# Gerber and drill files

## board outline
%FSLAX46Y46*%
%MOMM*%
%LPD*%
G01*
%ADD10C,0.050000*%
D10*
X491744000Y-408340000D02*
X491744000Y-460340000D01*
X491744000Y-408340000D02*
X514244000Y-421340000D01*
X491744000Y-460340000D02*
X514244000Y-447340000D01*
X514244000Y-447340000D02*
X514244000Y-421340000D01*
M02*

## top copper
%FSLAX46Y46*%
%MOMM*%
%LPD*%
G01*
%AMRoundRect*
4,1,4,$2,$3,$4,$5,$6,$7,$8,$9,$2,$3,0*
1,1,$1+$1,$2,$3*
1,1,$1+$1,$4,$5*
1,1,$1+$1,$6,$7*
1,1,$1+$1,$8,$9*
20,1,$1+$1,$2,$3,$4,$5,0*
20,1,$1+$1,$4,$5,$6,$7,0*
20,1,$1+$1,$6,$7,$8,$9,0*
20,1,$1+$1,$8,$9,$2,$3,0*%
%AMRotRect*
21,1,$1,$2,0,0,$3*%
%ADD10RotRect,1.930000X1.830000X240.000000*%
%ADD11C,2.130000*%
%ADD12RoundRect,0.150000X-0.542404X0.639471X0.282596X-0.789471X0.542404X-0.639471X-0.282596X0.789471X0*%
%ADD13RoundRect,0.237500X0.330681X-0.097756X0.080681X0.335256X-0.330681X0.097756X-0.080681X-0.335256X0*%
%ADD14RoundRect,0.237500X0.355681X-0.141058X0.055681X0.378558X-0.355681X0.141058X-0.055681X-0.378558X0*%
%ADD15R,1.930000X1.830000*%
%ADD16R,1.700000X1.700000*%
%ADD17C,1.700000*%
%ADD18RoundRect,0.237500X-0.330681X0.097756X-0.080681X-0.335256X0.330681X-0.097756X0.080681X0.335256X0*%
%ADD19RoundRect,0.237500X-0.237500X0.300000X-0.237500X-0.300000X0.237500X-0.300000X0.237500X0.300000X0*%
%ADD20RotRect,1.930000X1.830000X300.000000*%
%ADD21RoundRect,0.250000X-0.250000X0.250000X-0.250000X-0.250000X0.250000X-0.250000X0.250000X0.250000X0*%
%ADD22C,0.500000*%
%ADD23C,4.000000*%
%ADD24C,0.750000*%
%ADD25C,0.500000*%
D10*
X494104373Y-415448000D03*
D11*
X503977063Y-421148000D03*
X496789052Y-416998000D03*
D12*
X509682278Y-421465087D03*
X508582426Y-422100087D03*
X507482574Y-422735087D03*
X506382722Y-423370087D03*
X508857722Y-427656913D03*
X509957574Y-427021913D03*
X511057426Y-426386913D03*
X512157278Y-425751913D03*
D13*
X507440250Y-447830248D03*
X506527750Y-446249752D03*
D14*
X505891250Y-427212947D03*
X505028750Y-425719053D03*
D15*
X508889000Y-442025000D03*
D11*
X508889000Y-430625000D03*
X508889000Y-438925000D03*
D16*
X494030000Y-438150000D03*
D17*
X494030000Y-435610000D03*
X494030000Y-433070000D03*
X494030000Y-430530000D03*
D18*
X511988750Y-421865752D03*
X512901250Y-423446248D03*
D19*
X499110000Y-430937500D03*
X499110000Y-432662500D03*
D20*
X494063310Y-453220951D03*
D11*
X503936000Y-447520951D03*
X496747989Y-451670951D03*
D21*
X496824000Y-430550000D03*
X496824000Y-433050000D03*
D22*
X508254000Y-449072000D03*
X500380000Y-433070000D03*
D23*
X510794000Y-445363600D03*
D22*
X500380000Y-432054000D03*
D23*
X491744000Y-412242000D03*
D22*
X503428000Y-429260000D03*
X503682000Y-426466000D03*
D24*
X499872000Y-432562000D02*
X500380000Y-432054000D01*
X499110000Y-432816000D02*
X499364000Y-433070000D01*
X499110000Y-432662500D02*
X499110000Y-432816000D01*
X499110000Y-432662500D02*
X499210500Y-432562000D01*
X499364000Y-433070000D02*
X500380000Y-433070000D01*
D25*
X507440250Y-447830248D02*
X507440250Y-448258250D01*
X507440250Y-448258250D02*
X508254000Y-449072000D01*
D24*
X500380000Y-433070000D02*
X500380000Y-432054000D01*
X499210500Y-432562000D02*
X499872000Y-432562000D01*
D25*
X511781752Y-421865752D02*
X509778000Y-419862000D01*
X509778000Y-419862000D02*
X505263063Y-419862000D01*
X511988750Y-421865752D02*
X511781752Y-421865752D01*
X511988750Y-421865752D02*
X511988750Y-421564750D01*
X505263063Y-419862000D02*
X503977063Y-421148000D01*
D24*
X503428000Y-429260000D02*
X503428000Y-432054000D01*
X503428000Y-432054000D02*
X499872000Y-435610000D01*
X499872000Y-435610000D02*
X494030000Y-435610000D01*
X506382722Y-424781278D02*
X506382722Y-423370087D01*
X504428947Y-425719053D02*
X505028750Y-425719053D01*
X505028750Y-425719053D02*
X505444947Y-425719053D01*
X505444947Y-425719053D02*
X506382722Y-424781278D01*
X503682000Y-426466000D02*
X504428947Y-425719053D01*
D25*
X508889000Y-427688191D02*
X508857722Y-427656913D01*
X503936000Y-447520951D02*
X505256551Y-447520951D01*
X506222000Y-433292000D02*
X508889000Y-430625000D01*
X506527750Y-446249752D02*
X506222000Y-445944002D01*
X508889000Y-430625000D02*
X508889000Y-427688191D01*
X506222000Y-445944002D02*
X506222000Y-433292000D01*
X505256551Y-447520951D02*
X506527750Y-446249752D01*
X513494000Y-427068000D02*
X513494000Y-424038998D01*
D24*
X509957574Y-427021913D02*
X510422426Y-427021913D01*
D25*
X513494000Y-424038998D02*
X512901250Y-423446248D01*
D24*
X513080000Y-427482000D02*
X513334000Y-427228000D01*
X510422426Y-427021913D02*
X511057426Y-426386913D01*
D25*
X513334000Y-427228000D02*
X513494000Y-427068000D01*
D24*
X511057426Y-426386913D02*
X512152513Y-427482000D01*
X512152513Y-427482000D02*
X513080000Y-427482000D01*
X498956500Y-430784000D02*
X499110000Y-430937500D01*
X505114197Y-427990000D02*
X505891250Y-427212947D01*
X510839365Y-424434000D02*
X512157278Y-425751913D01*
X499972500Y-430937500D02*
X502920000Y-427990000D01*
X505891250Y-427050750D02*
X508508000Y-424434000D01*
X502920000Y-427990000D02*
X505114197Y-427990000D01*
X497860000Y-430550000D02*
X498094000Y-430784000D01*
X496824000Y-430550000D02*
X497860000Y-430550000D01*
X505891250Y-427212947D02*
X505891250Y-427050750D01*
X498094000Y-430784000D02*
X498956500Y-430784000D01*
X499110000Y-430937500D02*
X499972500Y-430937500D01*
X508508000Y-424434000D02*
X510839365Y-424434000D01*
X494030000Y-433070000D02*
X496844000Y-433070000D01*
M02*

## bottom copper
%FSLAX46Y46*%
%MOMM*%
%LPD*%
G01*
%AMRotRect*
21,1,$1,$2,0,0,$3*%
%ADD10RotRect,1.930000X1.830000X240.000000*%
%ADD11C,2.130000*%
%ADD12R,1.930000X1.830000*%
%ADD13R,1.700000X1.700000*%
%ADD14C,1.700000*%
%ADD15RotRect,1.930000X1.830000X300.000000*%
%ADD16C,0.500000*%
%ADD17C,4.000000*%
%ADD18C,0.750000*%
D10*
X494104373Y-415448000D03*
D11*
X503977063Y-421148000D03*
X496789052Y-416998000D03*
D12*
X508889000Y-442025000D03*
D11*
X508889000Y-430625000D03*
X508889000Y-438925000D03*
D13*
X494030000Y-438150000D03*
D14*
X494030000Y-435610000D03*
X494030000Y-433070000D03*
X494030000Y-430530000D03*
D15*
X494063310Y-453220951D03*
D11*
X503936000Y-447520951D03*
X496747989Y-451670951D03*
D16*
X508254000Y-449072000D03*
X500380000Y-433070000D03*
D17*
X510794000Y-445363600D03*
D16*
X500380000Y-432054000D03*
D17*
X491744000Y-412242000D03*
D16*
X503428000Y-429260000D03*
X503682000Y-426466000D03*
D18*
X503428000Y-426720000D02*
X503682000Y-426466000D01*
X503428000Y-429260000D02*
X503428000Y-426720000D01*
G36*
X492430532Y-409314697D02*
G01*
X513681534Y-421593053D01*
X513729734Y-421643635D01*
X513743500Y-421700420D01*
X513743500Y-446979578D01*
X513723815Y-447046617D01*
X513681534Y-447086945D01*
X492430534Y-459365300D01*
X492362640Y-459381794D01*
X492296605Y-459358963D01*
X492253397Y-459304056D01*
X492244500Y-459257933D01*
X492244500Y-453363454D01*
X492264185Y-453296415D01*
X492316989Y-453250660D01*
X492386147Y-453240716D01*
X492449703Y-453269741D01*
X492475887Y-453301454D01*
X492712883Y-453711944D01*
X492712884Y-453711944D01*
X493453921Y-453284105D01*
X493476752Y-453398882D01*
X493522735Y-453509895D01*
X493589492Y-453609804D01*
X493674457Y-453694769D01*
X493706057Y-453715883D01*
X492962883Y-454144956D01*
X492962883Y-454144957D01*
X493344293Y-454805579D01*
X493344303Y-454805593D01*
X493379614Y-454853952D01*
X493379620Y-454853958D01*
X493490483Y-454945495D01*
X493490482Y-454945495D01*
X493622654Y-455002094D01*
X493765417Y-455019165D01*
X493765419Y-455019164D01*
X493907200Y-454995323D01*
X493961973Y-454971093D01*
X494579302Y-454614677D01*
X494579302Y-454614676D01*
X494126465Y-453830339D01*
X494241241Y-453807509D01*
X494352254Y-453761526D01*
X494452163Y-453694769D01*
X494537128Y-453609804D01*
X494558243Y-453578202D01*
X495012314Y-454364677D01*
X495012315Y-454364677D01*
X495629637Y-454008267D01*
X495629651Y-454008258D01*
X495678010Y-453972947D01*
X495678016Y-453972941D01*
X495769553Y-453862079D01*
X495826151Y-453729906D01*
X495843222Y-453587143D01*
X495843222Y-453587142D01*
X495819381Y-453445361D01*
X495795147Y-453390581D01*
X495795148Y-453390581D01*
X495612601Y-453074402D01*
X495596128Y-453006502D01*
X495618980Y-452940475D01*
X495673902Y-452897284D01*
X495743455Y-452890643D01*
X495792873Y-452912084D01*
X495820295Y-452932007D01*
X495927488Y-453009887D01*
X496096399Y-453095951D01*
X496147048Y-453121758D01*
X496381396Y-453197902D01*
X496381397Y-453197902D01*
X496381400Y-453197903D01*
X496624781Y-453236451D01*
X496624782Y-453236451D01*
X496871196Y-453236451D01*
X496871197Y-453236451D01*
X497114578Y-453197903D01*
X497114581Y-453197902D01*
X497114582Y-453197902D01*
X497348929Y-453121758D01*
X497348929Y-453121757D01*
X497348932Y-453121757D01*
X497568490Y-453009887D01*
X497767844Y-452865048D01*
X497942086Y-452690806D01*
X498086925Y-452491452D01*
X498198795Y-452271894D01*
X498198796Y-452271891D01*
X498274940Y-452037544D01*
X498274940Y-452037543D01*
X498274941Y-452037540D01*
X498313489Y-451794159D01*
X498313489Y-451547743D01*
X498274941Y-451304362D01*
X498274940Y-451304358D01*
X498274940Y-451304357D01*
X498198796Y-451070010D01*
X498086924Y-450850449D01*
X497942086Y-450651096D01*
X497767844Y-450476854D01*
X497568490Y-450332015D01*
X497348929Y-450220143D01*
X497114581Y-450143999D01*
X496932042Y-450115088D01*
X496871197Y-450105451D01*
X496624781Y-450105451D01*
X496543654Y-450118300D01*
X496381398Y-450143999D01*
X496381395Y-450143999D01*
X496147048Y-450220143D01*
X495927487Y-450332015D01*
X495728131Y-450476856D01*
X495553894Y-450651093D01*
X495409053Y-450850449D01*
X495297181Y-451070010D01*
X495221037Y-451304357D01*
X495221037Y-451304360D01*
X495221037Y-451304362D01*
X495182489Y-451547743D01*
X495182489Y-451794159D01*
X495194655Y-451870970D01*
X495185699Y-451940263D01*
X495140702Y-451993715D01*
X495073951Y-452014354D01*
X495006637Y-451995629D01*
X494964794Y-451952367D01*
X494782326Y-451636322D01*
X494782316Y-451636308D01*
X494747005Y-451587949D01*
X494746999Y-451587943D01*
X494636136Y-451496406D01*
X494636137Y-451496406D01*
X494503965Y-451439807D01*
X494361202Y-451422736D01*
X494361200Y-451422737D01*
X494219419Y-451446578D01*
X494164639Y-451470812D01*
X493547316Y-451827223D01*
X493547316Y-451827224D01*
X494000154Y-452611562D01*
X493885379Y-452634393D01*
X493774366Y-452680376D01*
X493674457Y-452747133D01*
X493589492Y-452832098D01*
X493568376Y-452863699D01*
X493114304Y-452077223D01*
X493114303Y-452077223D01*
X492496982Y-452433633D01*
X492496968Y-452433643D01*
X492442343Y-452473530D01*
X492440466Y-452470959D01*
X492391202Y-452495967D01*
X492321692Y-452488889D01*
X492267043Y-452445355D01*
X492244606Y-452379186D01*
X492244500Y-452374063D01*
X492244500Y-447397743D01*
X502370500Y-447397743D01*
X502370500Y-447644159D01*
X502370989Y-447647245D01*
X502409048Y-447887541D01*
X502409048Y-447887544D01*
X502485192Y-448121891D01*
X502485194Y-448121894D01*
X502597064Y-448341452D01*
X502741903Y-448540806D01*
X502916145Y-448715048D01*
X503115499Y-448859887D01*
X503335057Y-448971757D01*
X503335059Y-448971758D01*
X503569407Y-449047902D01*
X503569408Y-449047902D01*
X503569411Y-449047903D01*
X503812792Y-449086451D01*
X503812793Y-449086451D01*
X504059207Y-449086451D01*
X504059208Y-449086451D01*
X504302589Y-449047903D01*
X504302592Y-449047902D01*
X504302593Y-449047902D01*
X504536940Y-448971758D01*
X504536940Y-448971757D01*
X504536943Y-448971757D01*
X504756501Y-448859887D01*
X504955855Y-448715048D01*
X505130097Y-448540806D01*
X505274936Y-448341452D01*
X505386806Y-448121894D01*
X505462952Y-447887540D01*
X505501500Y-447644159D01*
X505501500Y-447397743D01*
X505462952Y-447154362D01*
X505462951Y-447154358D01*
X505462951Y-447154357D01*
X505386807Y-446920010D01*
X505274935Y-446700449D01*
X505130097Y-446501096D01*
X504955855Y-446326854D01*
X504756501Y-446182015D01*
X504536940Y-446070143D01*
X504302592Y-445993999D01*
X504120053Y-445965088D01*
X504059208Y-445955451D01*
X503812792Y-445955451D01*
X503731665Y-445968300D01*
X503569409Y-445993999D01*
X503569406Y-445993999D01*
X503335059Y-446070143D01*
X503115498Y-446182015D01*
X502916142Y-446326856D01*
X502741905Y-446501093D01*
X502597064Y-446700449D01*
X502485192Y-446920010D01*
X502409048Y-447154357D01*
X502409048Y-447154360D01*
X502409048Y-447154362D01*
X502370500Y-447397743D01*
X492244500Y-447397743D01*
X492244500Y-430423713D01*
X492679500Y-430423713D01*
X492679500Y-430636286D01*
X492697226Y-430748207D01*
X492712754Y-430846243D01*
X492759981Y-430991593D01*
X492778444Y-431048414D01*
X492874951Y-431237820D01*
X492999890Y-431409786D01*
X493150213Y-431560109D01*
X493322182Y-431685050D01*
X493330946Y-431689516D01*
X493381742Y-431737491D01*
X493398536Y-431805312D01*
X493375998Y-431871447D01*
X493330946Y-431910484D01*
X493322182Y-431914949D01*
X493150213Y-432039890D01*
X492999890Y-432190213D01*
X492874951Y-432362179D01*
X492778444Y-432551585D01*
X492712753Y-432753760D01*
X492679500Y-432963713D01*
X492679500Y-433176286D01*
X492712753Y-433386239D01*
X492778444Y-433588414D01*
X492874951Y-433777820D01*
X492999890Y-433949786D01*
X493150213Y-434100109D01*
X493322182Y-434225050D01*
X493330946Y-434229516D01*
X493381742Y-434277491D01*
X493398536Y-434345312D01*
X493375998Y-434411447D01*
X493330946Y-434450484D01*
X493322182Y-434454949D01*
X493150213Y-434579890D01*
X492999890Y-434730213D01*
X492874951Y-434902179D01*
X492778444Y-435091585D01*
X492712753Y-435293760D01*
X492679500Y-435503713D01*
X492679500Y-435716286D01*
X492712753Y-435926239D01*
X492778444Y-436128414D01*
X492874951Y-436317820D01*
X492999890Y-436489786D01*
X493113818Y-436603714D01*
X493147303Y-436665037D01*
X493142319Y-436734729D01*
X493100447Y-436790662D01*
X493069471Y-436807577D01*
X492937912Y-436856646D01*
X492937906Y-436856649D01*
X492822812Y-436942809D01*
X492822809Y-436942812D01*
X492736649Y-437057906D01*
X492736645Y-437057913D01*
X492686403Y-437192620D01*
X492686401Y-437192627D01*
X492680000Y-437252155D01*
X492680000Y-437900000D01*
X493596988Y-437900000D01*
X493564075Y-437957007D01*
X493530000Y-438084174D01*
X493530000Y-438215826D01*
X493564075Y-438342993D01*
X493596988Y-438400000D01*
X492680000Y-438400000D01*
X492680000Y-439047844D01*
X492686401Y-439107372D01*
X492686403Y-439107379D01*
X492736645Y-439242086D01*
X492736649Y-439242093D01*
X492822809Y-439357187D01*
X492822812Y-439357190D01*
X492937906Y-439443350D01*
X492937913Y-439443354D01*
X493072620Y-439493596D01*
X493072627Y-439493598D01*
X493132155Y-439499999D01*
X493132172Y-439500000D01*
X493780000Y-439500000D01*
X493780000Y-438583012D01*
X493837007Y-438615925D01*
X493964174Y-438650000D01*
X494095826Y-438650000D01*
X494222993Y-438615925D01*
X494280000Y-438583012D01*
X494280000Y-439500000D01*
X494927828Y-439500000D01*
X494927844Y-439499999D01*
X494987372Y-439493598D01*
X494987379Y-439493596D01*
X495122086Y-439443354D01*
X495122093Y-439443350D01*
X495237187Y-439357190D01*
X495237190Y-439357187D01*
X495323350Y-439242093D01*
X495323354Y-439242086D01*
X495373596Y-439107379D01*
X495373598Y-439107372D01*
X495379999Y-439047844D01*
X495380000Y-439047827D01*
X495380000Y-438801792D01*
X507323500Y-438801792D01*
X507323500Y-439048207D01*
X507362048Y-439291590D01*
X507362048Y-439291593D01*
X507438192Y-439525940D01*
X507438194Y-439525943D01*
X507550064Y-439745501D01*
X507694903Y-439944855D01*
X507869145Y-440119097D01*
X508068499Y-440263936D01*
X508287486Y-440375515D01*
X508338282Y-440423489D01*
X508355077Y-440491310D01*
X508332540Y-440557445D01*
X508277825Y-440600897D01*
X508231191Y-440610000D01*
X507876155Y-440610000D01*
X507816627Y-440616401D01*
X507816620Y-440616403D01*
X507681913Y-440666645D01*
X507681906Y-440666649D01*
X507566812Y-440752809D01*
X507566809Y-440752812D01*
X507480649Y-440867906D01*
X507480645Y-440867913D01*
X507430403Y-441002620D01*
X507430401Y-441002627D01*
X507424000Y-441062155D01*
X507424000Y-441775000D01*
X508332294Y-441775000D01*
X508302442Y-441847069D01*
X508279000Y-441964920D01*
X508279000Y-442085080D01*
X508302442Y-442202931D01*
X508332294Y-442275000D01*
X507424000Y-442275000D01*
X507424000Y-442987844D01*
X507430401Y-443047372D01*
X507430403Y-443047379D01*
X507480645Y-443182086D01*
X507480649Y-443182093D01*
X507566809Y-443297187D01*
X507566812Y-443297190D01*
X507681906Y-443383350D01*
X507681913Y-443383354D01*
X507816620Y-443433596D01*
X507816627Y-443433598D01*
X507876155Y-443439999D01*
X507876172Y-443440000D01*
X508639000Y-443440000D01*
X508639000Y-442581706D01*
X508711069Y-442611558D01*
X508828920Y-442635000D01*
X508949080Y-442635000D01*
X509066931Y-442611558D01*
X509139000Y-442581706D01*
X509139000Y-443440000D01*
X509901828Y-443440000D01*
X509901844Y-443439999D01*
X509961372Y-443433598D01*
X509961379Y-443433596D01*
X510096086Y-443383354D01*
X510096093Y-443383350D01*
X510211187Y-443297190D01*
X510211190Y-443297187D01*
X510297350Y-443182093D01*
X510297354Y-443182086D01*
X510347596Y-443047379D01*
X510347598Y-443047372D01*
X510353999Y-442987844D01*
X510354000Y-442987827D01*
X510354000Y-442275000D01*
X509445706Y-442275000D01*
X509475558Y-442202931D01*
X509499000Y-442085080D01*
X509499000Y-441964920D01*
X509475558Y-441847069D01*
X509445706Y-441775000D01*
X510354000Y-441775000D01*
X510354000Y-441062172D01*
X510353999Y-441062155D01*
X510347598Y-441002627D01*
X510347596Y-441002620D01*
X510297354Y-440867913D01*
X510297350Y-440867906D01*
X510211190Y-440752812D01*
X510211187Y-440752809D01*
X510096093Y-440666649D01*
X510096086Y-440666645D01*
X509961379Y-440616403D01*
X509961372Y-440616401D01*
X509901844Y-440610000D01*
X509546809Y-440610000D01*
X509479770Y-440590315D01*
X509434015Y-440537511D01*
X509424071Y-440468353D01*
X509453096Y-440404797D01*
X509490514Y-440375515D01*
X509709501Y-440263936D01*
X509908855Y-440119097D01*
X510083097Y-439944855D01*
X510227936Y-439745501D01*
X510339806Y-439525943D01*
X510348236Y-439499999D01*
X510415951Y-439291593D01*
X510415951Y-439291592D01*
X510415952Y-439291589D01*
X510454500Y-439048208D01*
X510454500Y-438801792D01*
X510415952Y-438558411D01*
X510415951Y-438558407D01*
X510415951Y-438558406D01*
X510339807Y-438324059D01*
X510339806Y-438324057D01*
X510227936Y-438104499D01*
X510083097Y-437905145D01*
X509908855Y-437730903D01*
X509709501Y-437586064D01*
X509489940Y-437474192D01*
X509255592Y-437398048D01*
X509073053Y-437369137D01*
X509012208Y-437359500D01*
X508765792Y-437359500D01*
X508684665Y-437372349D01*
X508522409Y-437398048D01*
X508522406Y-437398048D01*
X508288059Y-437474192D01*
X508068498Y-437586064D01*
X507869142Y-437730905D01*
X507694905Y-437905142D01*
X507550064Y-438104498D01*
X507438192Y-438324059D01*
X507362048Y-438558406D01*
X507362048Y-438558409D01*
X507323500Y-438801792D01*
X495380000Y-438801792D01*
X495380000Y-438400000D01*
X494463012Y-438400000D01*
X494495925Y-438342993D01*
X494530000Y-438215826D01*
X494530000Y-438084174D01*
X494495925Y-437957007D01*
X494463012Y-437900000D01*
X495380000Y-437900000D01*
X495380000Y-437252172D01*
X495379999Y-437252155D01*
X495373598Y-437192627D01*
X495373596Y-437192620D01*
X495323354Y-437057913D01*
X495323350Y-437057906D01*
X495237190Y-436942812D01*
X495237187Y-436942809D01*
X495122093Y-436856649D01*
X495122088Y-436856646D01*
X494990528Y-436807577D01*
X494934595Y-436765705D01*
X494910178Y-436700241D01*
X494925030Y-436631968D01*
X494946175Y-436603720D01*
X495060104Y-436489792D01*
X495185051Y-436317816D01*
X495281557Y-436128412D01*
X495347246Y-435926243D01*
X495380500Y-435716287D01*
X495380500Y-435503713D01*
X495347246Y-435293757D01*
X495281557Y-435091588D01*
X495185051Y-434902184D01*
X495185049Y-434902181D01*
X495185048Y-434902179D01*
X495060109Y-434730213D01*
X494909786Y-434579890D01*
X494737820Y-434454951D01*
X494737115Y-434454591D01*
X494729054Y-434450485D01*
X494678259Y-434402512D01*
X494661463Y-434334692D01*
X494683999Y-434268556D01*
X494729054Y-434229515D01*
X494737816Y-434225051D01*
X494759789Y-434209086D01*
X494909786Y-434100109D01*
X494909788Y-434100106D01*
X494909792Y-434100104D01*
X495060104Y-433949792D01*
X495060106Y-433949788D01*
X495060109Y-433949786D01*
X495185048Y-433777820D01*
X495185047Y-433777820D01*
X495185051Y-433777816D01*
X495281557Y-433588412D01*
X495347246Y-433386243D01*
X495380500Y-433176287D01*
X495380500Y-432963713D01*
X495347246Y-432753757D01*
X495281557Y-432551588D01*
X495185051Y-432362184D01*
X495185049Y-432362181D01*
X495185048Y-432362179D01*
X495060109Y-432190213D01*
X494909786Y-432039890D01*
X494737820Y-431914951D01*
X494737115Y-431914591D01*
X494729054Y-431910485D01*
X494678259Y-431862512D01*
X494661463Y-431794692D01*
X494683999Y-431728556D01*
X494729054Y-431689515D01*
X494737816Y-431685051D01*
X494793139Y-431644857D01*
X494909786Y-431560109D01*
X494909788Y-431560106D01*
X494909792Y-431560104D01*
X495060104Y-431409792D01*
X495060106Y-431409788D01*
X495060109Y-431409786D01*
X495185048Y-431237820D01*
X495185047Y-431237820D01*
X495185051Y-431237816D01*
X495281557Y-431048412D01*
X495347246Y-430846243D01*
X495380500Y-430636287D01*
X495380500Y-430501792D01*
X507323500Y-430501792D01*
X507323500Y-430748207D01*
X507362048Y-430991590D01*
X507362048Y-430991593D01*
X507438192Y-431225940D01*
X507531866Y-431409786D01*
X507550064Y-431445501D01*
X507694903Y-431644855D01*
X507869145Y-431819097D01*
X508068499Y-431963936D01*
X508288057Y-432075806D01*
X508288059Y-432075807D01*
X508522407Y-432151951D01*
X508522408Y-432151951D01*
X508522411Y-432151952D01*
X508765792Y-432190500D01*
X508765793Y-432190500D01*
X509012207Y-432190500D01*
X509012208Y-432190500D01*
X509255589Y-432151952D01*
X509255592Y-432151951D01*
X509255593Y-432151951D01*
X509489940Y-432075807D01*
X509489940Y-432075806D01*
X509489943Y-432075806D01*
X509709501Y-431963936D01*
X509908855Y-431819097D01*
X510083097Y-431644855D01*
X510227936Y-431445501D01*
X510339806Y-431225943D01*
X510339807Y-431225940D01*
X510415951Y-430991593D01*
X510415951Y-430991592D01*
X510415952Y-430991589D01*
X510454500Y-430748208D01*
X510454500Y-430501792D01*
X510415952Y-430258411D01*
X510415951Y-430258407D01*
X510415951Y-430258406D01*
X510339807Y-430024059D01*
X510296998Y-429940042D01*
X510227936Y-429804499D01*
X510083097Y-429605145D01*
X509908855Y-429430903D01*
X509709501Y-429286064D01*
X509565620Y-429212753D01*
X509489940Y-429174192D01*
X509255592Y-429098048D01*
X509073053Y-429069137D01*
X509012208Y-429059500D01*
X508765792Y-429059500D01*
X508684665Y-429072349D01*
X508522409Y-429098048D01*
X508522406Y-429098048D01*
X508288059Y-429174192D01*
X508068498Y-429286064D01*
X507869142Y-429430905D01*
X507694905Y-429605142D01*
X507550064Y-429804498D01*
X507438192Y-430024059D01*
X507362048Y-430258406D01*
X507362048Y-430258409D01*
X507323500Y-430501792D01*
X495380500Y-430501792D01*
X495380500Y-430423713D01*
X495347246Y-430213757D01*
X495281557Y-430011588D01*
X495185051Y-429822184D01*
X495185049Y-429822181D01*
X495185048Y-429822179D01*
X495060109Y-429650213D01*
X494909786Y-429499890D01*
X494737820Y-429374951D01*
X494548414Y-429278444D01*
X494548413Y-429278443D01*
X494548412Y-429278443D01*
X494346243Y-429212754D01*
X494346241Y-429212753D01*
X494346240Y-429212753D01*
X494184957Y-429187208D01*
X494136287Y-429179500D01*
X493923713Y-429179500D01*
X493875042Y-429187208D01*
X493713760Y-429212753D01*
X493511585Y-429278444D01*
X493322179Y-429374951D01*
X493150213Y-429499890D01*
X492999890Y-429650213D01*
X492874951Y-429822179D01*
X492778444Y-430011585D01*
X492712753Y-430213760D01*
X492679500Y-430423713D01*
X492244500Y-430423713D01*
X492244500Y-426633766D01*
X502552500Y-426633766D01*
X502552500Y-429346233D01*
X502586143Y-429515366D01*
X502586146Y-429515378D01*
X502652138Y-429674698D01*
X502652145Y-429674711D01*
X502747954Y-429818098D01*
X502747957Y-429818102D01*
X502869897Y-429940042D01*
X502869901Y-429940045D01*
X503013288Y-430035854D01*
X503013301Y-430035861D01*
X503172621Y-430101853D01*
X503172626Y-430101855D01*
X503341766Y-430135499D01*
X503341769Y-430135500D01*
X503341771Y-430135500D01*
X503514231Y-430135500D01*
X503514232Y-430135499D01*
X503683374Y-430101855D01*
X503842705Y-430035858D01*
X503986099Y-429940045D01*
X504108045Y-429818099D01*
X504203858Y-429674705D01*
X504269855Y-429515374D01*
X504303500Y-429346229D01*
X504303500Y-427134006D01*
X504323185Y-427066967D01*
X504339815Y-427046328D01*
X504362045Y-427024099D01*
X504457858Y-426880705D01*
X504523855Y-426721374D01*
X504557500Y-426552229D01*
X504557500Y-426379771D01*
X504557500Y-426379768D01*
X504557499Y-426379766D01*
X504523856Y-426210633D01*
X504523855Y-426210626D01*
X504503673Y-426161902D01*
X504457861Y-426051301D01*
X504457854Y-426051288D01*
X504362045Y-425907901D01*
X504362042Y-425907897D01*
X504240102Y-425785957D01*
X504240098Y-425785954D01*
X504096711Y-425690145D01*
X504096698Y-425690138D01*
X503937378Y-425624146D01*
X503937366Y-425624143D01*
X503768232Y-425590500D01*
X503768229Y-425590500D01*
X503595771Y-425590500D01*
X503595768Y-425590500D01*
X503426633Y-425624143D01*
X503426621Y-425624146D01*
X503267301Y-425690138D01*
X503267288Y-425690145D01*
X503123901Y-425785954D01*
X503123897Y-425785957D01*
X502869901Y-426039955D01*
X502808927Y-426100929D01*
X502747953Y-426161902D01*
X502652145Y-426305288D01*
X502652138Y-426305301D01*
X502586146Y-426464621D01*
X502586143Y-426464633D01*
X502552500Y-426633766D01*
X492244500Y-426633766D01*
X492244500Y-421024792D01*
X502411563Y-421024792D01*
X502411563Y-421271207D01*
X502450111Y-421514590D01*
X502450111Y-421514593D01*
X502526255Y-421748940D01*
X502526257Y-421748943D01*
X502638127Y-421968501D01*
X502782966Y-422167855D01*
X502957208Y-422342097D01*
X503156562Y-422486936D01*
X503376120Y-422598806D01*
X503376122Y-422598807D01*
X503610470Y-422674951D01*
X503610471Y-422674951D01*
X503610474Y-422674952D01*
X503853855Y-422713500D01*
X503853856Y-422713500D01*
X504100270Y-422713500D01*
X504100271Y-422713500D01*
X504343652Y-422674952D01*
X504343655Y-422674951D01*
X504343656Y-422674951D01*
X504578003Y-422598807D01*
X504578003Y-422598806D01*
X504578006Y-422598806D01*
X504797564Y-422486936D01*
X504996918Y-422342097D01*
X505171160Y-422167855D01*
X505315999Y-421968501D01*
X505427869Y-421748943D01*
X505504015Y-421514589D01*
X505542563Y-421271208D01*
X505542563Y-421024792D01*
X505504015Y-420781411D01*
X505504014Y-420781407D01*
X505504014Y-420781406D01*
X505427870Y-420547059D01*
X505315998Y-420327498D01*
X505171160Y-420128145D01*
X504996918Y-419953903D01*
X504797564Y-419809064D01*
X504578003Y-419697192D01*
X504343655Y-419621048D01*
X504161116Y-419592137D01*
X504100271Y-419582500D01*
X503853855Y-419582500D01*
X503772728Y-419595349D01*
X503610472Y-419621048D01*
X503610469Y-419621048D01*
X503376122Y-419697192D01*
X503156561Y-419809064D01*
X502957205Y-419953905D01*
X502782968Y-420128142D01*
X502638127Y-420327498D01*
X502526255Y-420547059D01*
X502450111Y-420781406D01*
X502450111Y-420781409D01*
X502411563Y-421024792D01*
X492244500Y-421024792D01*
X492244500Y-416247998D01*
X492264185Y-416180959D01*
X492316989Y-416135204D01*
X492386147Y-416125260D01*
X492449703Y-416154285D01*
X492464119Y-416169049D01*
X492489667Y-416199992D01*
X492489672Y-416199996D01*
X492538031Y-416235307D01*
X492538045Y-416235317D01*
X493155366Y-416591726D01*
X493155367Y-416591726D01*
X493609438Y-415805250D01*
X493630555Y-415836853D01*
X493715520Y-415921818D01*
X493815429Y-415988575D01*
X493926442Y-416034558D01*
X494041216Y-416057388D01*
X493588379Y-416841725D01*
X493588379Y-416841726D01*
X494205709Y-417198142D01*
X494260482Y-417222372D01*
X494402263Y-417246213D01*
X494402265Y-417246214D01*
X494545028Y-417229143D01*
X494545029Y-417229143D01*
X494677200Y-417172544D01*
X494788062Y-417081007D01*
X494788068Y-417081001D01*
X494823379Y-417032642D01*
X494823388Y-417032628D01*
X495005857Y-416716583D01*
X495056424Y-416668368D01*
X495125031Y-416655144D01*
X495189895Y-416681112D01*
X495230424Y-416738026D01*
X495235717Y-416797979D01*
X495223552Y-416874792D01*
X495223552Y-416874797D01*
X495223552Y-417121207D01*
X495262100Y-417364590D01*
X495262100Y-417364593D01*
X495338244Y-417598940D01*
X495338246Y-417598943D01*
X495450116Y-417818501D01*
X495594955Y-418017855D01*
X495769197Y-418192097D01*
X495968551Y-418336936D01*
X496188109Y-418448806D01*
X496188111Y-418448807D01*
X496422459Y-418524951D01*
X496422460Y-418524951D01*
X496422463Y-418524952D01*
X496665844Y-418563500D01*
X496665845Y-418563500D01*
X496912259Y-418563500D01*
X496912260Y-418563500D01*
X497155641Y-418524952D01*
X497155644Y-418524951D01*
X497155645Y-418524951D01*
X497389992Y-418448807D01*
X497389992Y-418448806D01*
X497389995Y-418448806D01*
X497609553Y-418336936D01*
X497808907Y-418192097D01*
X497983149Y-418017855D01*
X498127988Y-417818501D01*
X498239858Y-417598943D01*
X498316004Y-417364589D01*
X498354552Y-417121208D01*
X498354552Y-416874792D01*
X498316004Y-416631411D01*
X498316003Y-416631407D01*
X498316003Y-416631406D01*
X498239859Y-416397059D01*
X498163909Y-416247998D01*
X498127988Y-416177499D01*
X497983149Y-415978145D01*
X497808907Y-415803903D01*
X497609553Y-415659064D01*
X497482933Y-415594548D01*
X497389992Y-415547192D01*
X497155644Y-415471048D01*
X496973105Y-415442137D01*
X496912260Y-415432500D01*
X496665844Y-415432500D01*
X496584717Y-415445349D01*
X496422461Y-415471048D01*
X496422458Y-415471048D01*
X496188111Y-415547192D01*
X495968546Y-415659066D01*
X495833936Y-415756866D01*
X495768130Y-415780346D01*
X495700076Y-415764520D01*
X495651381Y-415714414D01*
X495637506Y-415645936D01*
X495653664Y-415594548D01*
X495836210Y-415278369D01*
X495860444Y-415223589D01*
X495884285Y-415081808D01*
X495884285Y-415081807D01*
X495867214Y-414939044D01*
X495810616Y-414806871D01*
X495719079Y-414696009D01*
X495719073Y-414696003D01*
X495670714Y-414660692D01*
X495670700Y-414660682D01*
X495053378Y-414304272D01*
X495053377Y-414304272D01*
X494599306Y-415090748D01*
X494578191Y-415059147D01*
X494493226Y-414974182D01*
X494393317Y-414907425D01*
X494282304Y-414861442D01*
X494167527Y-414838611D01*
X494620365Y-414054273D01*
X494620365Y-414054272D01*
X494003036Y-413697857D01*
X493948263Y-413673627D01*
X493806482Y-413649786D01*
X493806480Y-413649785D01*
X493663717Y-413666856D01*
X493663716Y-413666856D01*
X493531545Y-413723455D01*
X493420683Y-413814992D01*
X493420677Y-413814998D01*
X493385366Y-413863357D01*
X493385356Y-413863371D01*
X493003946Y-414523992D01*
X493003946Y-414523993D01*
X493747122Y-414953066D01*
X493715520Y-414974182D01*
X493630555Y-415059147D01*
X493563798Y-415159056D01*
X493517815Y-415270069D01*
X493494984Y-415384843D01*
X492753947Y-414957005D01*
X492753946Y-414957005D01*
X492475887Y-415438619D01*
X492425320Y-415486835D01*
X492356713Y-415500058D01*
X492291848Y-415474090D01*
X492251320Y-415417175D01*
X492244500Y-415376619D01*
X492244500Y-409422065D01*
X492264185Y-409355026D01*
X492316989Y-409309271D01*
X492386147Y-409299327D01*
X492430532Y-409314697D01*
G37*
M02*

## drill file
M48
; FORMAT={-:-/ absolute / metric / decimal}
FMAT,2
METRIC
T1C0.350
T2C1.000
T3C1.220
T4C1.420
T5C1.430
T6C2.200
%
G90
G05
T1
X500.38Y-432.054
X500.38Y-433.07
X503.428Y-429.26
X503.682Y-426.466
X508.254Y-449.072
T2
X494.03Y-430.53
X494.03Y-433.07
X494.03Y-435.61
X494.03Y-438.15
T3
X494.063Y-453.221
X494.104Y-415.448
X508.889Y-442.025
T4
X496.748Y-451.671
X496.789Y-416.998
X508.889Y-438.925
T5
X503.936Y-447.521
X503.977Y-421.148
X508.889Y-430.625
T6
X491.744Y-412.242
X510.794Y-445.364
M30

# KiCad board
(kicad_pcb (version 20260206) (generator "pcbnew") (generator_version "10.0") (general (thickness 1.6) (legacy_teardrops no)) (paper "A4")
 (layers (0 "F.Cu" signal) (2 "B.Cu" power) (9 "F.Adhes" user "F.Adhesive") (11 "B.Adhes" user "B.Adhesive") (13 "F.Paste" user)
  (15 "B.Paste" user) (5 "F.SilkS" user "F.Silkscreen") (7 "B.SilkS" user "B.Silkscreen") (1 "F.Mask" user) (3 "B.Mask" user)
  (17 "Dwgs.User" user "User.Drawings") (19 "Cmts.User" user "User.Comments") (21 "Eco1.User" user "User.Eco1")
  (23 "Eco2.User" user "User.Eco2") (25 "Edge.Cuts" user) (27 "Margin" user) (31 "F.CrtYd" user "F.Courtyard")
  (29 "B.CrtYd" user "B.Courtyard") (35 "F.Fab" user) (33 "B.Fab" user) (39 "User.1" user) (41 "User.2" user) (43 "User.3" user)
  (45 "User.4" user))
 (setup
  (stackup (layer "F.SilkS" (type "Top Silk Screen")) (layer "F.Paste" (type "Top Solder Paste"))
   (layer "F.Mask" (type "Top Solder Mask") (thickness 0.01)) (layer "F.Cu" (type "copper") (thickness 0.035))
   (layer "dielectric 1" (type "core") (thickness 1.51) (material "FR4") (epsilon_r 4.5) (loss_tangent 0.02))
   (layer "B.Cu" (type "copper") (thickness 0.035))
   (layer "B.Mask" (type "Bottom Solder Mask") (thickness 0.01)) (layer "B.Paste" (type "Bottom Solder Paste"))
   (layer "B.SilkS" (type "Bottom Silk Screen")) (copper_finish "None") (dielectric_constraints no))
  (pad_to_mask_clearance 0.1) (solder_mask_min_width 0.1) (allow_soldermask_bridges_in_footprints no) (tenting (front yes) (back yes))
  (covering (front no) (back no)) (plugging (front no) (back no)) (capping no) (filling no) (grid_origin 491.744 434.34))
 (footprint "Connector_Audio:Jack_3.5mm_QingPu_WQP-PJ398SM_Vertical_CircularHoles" (layer "F.Cu") (at 494.104373 415.448 60)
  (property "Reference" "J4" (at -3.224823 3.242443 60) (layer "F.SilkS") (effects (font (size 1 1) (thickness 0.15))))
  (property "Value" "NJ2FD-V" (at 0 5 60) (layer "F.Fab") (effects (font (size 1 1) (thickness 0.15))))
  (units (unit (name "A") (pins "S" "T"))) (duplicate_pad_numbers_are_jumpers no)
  (pad "S" thru_hole rect (at 0 0 240) (size 1.93 1.83) (drill 1.22) (layers "*.Cu" "*.Mask") (remove_unused_layers no) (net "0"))
  (pad "T" thru_hole circle (at 0 11.4 240) (size 2.13 2.13) (drill 1.43) (layers "*.Cu" "*.Mask") (remove_unused_layers no)
   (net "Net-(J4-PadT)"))
  (pad "TN" thru_hole circle (at 0 3.1 240) (size 2.13 2.13) (drill 1.42) (layers "*.Cu" "*.Mask") (remove_unused_layers no))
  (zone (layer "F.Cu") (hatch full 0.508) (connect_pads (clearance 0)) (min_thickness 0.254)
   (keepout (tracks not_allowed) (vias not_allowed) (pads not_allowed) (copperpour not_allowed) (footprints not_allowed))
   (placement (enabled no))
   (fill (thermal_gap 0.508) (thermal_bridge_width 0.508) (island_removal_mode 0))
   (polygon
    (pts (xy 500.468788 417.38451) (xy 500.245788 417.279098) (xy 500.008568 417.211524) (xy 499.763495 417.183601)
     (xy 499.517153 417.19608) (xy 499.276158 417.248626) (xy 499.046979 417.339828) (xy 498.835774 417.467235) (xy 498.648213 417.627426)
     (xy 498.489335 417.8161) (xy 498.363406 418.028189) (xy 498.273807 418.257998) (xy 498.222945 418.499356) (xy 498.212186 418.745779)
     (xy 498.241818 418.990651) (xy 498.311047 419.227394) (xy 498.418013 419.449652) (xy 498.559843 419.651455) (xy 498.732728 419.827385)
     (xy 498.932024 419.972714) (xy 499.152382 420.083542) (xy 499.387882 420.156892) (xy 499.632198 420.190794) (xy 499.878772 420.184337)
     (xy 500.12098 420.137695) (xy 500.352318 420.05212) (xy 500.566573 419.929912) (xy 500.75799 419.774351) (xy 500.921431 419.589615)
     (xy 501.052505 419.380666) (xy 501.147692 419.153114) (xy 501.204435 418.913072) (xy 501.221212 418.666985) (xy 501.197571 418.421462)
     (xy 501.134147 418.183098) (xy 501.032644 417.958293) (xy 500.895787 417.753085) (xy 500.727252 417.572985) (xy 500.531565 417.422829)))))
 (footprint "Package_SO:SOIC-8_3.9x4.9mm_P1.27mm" (layer "F.Cu") (at 509.27 424.561 -60)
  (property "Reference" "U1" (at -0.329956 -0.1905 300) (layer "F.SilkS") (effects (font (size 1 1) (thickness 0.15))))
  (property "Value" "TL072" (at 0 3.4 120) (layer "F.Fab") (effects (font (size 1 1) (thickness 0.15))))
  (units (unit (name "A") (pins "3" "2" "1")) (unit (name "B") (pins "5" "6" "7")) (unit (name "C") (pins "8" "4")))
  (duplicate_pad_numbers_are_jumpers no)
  (pad "1" smd roundrect (at -2.475 -1.905 300) (size 1.95 0.6) (layers "F.Cu" "F.Mask" "F.Paste") (roundrect_rratio 0.25))
  (pad "2" smd roundrect (at -2.475 -0.635 300) (size 1.95 0.6) (layers "F.Cu" "F.Mask" "F.Paste") (roundrect_rratio 0.25))
  (pad "3" smd roundrect (at -2.475 0.635 300) (size 1.95 0.6) (layers "F.Cu" "F.Mask" "F.Paste") (roundrect_rratio 0.25))
  (pad "4" smd roundrect (at -2.475 1.905 300) (size 1.95 0.6) (layers "F.Cu" "F.Mask" "F.Paste") (roundrect_rratio 0.25) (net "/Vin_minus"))
  (pad "5" smd roundrect (at 2.475 1.905 300) (size 1.95 0.6) (layers "F.Cu" "F.Mask" "F.Paste") (roundrect_rratio 0.25) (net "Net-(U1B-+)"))
  (pad "6" smd roundrect (at 2.475 0.635 300) (size 1.95 0.6) (layers "F.Cu" "F.Mask" "F.Paste") (roundrect_rratio 0.25) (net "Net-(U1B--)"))
  (pad "7" smd roundrect (at 2.475 -0.635 300) (size 1.95 0.6) (layers "F.Cu" "F.Mask" "F.Paste") (roundrect_rratio 0.25)
   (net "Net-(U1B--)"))
  (pad "8" smd roundrect (at 2.475 -1.905 300) (size 1.95 0.6) (layers "F.Cu" "F.Mask" "F.Paste") (roundrect_rratio 0.25) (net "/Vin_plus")))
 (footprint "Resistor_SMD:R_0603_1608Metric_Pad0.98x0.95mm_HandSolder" (layer "F.Cu") (at 506.984 447.04 120)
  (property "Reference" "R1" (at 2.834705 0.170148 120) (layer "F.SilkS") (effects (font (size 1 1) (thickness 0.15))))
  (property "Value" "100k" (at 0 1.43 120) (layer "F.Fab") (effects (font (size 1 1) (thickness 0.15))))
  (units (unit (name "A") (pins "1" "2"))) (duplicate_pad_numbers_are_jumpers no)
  (pad "1" smd roundrect (at -0.9125 0 120) (size 0.975 0.95) (layers "F.Cu" "F.Mask" "F.Paste") (roundrect_rratio 0.25) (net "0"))
  (pad "2" smd roundrect (at 0.9125 0 120) (size 0.975 0.95) (layers "F.Cu" "F.Mask" "F.Paste") (roundrect_rratio 0.25) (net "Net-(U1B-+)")))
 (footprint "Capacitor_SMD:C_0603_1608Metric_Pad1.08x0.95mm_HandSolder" (layer "F.Cu") (at 505.46 426.466 120)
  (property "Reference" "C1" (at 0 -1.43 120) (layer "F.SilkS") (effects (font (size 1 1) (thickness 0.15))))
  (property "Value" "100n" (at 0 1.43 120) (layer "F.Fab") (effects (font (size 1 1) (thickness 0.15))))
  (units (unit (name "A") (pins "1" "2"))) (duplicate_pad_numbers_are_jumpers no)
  (pad "1" smd roundrect (at -0.8625 0 120) (size 1.075 0.95) (layers "F.Cu" "F.Mask" "F.Paste") (roundrect_rratio 0.25) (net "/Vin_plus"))
  (pad "2" smd roundrect (at 0.8625 0 120) (size 1.075 0.95) (layers "F.Cu" "F.Mask" "F.Paste") (roundrect_rratio 0.25) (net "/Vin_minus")))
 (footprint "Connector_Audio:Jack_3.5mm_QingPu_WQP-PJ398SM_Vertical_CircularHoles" (layer "F.Cu") (at 508.889 442.025 180)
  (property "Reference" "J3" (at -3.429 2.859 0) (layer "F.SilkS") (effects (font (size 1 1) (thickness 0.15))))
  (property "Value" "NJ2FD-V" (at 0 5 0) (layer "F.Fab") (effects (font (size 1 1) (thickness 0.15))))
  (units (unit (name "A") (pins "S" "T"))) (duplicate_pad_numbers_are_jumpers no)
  (pad "S" thru_hole rect (at 0 0) (size 1.93 1.83) (drill 1.22) (layers "*.Cu" "*.Mask") (remove_unused_layers no) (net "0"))
  (pad "T" thru_hole circle (at 0 11.4) (size 2.13 2.13) (drill 1.43) (layers "*.Cu" "*.Mask") (remove_unused_layers no) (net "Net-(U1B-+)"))
  (pad "TN" thru_hole circle (at 0 3.1) (size 2.13 2.13) (drill 1.42) (layers "*.Cu" "*.Mask") (remove_unused_layers no))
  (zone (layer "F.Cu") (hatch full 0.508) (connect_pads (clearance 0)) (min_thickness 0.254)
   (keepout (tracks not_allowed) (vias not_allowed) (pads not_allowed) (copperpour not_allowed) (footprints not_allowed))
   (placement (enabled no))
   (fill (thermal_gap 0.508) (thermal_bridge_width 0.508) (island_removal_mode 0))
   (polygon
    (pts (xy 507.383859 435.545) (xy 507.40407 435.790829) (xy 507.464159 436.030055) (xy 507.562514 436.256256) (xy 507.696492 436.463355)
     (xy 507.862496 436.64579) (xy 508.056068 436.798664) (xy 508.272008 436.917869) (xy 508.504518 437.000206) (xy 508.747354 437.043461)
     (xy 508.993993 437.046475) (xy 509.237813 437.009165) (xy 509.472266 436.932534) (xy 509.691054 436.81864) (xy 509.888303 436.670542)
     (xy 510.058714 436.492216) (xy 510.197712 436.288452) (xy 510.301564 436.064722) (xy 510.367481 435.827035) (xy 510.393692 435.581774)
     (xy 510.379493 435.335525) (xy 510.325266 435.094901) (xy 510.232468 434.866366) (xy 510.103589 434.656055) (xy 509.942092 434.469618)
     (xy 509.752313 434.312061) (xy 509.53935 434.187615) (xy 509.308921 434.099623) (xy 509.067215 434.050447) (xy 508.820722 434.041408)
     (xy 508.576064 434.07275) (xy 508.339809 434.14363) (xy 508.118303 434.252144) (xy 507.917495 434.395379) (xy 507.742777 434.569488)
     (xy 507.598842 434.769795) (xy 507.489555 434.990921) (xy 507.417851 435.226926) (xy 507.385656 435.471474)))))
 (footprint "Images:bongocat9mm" (layer "F.Cu") (at 497.367634 444.023144 30)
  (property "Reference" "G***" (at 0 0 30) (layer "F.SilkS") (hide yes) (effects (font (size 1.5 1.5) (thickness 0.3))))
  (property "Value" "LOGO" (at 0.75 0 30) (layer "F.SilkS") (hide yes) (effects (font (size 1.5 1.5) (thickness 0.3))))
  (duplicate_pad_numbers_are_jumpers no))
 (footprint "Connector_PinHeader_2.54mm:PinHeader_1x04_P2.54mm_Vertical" (layer "F.Cu") (at 494.03 438.15 180)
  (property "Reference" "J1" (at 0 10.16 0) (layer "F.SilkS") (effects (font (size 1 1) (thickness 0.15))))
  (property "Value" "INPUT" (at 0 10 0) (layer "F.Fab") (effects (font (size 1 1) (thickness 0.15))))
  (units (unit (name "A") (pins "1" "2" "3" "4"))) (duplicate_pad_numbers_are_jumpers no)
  (pad "1" thru_hole rect (at 0 0 180) (size 1.7 1.7) (drill 1) (layers "*.Cu" "*.Mask") (remove_unused_layers no) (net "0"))
  (pad "2" thru_hole circle (at 0 2.54 180) (size 1.7 1.7) (drill 1) (layers "*.Cu" "*.Mask") (remove_unused_layers no) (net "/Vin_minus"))
  (pad "3" thru_hole circle (at 0 5.08 180) (size 1.7 1.7) (drill 1) (layers "*.Cu" "*.Mask") (remove_unused_layers no) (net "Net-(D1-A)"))
  (pad "4" thru_hole circle (at 0 7.62 180) (size 1.7 1.7) (drill 1) (layers "*.Cu" "*.Mask") (remove_unused_layers no) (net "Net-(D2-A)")))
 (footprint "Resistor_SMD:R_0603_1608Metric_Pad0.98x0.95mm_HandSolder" (layer "F.Cu") (at 512.445 422.656 -60)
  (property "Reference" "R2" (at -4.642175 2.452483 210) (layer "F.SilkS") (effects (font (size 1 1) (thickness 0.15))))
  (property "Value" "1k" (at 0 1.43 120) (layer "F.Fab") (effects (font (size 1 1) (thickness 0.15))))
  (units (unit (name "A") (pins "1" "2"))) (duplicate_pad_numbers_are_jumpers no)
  (pad "1" smd roundrect (at -0.9125 0 300) (size 0.975 0.95) (layers "F.Cu" "F.Mask" "F.Paste") (roundrect_rratio 0.25)
   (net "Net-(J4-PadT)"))
  (pad "2" smd roundrect (at 0.9125 0 300) (size 0.975 0.95) (layers "F.Cu" "F.Mask" "F.Paste") (roundrect_rratio 0.25) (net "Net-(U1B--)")))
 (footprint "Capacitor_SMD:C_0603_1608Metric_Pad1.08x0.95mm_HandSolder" (layer "F.Cu") (at 499.11 431.8 -90)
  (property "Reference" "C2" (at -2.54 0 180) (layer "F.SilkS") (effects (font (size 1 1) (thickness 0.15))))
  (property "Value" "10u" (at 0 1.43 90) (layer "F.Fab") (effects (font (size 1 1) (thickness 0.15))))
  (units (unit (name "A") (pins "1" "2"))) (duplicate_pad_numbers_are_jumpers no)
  (pad "1" smd roundrect (at -0.8625 0 270) (size 1.075 0.95) (layers "F.Cu" "F.Mask" "F.Paste") (roundrect_rratio 0.25) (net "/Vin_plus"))
  (pad "2" smd roundrect (at 0.8625 0 270) (size 1.075 0.95) (layers "F.Cu" "F.Mask" "F.Paste") (roundrect_rratio 0.25) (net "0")))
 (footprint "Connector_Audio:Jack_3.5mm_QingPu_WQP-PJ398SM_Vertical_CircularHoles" (layer "F.Cu") (at 494.06331 453.220951 120)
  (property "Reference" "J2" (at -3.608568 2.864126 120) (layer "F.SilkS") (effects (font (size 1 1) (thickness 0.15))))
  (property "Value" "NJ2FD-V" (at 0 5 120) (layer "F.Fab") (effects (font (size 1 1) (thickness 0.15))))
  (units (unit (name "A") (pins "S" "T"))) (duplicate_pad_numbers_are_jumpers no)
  (pad "S" thru_hole rect (at 0 0 300) (size 1.93 1.83) (drill 1.22) (layers "*.Cu" "*.Mask") (remove_unused_layers no) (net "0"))
  (pad "T" thru_hole circle (at 0 11.4 300) (size 2.13 2.13) (drill 1.43) (layers "*.Cu" "*.Mask") (remove_unused_layers no)
   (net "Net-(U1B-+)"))
  (pad "TN" thru_hole circle (at 0 3.1 300) (size 2.13 2.13) (drill 1.42) (layers "*.Cu" "*.Mask") (remove_unused_layers no))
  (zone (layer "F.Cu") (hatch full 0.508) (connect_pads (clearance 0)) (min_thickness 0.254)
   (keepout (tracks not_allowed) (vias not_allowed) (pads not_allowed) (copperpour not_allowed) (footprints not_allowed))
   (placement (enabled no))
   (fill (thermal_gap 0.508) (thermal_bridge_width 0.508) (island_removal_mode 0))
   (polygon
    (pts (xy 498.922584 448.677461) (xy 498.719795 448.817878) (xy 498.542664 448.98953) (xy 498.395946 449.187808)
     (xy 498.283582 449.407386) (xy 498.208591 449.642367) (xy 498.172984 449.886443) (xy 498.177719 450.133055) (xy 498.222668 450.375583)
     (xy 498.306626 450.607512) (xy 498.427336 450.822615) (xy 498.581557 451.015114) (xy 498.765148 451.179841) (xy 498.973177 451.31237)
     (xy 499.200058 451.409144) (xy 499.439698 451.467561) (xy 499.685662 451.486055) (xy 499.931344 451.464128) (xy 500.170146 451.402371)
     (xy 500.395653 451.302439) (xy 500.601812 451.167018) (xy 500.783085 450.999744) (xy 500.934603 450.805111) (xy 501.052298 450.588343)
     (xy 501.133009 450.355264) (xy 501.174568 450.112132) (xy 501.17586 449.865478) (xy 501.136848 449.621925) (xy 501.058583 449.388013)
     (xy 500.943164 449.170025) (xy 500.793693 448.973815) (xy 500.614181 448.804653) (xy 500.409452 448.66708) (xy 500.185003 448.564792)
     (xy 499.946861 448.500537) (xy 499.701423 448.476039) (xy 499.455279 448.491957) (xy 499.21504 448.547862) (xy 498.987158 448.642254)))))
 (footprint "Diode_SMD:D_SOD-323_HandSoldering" (layer "F.Cu") (at 496.824 431.8 -90)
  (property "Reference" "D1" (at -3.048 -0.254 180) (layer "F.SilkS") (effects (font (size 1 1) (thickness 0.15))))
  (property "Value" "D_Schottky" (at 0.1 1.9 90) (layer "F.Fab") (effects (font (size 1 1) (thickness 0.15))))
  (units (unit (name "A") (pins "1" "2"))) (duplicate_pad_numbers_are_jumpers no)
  (pad "1" smd roundrect (at -1.25 0 270) (size 1 1) (layers "F.Cu" "F.Mask" "F.Paste") (roundrect_rratio 0.25) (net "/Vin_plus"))
  (pad "2" smd roundrect (at 1.25 0 270) (size 1 1) (layers "F.Cu" "F.Mask" "F.Paste") (roundrect_rratio 0.25) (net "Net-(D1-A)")))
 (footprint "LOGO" (layer "B.Cu") (at 498.094 444.754 180)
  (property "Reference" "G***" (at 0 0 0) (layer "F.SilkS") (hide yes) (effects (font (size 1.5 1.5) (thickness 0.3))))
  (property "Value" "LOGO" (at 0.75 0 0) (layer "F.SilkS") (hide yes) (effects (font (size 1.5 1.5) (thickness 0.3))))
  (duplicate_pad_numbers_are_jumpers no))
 (gr_line (start 491.744 408.34) (end 491.744 460.34) (stroke (width 0.05) (type default)) (layer "Edge.Cuts"))
 (gr_line (start 491.744 408.34) (end 514.244 421.34) (stroke (width 0.05) (type default)) (layer "Edge.Cuts"))
 (gr_line (start 491.744 460.34) (end 514.244 447.34) (stroke (width 0.05) (type default)) (layer "Edge.Cuts"))
 (gr_line (start 514.244 447.34) (end 514.244 421.34) (stroke (width 0.05) (type default)) (layer "Edge.Cuts"))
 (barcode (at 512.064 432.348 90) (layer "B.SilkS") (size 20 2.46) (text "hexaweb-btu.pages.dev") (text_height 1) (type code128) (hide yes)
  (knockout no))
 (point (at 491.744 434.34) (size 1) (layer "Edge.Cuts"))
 (segment (start 499.872 432.562) (end 500.38 432.054) (width 0.75) (layer "F.Cu") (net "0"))
 (segment (start 499.11 432.816) (end 499.364 433.07) (width 0.75) (layer "F.Cu") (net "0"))
 (segment (start 499.11 432.6625) (end 499.11 432.816) (width 0.75) (layer "F.Cu") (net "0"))
 (segment (start 499.11 432.6625) (end 499.2105 432.562) (width 0.75) (layer "F.Cu") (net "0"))
 (segment (start 499.364 433.07) (end 500.38 433.07) (width 0.75) (layer "F.Cu") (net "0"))
 (segment (start 507.44025 447.830248) (end 507.44025 448.25825) (width 0.5) (layer "F.Cu") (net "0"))
 (segment (start 507.44025 448.25825) (end 508.254 449.072) (width 0.5) (layer "F.Cu") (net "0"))
 (segment (start 500.38 433.07) (end 500.38 432.054) (width 0.75) (layer "F.Cu") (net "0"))
 (segment (start 499.2105 432.562) (end 499.872 432.562) (width 0.75) (layer "F.Cu") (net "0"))
 (via (at 508.254 449.072) (size 0.5) (drill 0.35) (layers "F.Cu" "B.Cu") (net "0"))
 (via (at 500.38 433.07) (size 0.5) (drill 0.35) (layers "F.Cu" "B.Cu") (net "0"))
 (via (at 510.794 445.3636) (size 4) (drill 2.2) (layers "F.Cu" "B.Cu") (free yes) (tenting (front no) (back no)) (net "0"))
 (via (at 500.38 432.054) (size 0.5) (drill 0.35) (layers "F.Cu" "B.Cu") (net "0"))
 (via (at 491.744 412.242) (size 4) (drill 2.2) (layers "F.Cu" "B.Cu") (free yes) (tenting (front no) (back no)) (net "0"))
 (segment (start 511.781752 421.865752) (end 509.778 419.862) (width 0.5) (layer "F.Cu") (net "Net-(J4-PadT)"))
 (segment (start 509.778 419.862) (end 505.263063 419.862) (width 0.5) (layer "F.Cu") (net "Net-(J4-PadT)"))
 (segment (start 511.98875 421.865752) (end 511.781752 421.865752) (width 0.5) (layer "F.Cu") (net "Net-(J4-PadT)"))
 (segment (start 511.98875 421.865752) (end 511.98875 421.56475) (width 0.5) (layer "F.Cu") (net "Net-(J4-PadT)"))
 (segment (start 505.263063 419.862) (end 503.977063 421.148) (width 0.5) (layer "F.Cu") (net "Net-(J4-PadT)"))
 (segment (start 503.428 429.26) (end 503.428 432.054) (width 0.75) (layer "F.Cu") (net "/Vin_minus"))
 (segment (start 503.428 432.054) (end 499.872 435.61) (width 0.75) (layer "F.Cu") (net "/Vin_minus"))
 (segment (start 499.872 435.61) (end 494.03 435.61) (width 0.75) (layer "F.Cu") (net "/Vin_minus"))
 (segment (start 506.382722 424.781278) (end 506.382722 423.370087) (width 0.75) (layer "F.Cu") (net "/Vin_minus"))
 (segment (start 504.428947 425.719053) (end 505.02875 425.719053) (width 0.75) (layer "F.Cu") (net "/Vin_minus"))
 (segment (start 505.02875 425.719053) (end 505.444947 425.719053) (width 0.75) (layer "F.Cu") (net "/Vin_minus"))
 (segment (start 505.444947 425.719053) (end 506.382722 424.781278) (width 0.75) (layer "F.Cu") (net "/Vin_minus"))
 (segment (start 503.682 426.466) (end 504.428947 425.719053) (width 0.75) (layer "F.Cu") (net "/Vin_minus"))
 (via (at 503.428 429.26) (size 0.5) (drill 0.35) (layers "F.Cu" "B.Cu") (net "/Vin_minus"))
 (via (at 503.682 426.466) (size 0.5) (drill 0.35) (layers "F.Cu" "B.Cu") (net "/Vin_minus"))
 (segment (start 503.428 426.72) (end 503.682 426.466) (width 0.75) (layer "B.Cu") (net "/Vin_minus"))
 (segment (start 503.428 429.26) (end 503.428 426.72) (width 0.75) (layer "B.Cu") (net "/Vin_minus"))
 (segment (start 508.889 427.688191) (end 508.857722 427.656913) (width 0.5) (layer "F.Cu") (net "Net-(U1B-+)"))
 (segment (start 503.936 447.520951) (end 505.256551 447.520951) (width 0.5) (layer "F.Cu") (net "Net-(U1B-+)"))
 (segment (start 506.222 433.292) (end 508.889 430.625) (width 0.5) (layer "F.Cu") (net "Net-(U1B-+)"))
 (segment (start 506.52775 446.249752) (end 506.222 445.944002) (width 0.5) (layer "F.Cu") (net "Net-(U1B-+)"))
 (segment (start 508.889 430.625) (end 508.889 427.688191) (width 0.5) (layer "F.Cu") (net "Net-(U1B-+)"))
 (segment (start 506.222 445.944002) (end 506.222 433.292) (width 0.5) (layer "F.Cu") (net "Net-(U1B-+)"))
 (segment (start 505.256551 447.520951) (end 506.52775 446.249752) (width 0.5) (layer "F.Cu") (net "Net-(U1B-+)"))
 (segment (start 513.494 427.068) (end 513.494 424.038998) (width 0.5) (layer "F.Cu") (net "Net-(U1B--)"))
 (segment (start 509.957574 427.021913) (end 510.422426 427.021913) (width 0.75) (layer "F.Cu") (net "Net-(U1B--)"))
 (segment (start 513.494 424.038998) (end 512.90125 423.446248) (width 0.5) (layer "F.Cu") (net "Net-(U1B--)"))
 (segment (start 513.08 427.482) (end 513.334 427.228) (width 0.75) (layer "F.Cu") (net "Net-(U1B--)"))
 (segment (start 510.422426 427.021913) (end 511.057426 426.386913) (width 0.75) (layer "F.Cu") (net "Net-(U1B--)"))
 (segment (start 513.334 427.228) (end 513.494 427.068) (width 0.5) (layer "F.Cu") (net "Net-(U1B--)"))
 (segment (start 511.057426 426.386913) (end 512.152513 427.482) (width 0.75) (layer "F.Cu") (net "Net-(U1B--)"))
 (segment (start 512.152513 427.482) (end 513.08 427.482) (width 0.75) (layer "F.Cu") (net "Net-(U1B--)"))
 (segment (start 498.9565 430.784) (end 499.11 430.9375) (width 0.75) (layer "F.Cu") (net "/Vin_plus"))
 (segment (start 505.114197 427.99) (end 505.89125 427.212947) (width 0.75) (layer "F.Cu") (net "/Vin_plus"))
 (segment (start 510.839365 424.434) (end 512.157278 425.751913) (width 0.75) (layer "F.Cu") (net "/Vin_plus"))
 (segment (start 499.9725 430.9375) (end 502.92 427.99) (width 0.75) (layer "F.Cu") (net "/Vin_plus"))
 (segment (start 505.89125 427.05075) (end 508.508 424.434) (width 0.75) (layer "F.Cu") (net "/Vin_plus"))
 (segment (start 502.92 427.99) (end 505.114197 427.99) (width 0.75) (layer "F.Cu") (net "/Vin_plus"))
 (segment (start 497.86 430.55) (end 498.094 430.784) (width 0.75) (layer "F.Cu") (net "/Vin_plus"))
 (segment (start 496.824 430.55) (end 497.86 430.55) (width 0.75) (layer "F.Cu") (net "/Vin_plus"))
 (segment (start 505.89125 427.212947) (end 505.89125 427.05075) (width 0.75) (layer "F.Cu") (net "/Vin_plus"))
 (segment (start 498.094 430.784) (end 498.9565 430.784) (width 0.75) (layer "F.Cu") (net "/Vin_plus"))
 (segment (start 499.11 430.9375) (end 499.9725 430.9375) (width 0.75) (layer "F.Cu") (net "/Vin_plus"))
 (segment (start 508.508 424.434) (end 510.839365 424.434) (width 0.75) (layer "F.Cu") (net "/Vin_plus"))
 (segment (start 494.03 433.07) (end 496.844 433.07) (width 0.75) (layer "F.Cu") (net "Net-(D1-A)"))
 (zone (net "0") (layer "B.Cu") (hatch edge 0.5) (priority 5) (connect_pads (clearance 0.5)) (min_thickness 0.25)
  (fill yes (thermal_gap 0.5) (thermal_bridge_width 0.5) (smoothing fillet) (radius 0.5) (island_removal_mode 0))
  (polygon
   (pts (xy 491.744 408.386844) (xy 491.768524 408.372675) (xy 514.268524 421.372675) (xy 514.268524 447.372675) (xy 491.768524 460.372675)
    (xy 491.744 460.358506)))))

